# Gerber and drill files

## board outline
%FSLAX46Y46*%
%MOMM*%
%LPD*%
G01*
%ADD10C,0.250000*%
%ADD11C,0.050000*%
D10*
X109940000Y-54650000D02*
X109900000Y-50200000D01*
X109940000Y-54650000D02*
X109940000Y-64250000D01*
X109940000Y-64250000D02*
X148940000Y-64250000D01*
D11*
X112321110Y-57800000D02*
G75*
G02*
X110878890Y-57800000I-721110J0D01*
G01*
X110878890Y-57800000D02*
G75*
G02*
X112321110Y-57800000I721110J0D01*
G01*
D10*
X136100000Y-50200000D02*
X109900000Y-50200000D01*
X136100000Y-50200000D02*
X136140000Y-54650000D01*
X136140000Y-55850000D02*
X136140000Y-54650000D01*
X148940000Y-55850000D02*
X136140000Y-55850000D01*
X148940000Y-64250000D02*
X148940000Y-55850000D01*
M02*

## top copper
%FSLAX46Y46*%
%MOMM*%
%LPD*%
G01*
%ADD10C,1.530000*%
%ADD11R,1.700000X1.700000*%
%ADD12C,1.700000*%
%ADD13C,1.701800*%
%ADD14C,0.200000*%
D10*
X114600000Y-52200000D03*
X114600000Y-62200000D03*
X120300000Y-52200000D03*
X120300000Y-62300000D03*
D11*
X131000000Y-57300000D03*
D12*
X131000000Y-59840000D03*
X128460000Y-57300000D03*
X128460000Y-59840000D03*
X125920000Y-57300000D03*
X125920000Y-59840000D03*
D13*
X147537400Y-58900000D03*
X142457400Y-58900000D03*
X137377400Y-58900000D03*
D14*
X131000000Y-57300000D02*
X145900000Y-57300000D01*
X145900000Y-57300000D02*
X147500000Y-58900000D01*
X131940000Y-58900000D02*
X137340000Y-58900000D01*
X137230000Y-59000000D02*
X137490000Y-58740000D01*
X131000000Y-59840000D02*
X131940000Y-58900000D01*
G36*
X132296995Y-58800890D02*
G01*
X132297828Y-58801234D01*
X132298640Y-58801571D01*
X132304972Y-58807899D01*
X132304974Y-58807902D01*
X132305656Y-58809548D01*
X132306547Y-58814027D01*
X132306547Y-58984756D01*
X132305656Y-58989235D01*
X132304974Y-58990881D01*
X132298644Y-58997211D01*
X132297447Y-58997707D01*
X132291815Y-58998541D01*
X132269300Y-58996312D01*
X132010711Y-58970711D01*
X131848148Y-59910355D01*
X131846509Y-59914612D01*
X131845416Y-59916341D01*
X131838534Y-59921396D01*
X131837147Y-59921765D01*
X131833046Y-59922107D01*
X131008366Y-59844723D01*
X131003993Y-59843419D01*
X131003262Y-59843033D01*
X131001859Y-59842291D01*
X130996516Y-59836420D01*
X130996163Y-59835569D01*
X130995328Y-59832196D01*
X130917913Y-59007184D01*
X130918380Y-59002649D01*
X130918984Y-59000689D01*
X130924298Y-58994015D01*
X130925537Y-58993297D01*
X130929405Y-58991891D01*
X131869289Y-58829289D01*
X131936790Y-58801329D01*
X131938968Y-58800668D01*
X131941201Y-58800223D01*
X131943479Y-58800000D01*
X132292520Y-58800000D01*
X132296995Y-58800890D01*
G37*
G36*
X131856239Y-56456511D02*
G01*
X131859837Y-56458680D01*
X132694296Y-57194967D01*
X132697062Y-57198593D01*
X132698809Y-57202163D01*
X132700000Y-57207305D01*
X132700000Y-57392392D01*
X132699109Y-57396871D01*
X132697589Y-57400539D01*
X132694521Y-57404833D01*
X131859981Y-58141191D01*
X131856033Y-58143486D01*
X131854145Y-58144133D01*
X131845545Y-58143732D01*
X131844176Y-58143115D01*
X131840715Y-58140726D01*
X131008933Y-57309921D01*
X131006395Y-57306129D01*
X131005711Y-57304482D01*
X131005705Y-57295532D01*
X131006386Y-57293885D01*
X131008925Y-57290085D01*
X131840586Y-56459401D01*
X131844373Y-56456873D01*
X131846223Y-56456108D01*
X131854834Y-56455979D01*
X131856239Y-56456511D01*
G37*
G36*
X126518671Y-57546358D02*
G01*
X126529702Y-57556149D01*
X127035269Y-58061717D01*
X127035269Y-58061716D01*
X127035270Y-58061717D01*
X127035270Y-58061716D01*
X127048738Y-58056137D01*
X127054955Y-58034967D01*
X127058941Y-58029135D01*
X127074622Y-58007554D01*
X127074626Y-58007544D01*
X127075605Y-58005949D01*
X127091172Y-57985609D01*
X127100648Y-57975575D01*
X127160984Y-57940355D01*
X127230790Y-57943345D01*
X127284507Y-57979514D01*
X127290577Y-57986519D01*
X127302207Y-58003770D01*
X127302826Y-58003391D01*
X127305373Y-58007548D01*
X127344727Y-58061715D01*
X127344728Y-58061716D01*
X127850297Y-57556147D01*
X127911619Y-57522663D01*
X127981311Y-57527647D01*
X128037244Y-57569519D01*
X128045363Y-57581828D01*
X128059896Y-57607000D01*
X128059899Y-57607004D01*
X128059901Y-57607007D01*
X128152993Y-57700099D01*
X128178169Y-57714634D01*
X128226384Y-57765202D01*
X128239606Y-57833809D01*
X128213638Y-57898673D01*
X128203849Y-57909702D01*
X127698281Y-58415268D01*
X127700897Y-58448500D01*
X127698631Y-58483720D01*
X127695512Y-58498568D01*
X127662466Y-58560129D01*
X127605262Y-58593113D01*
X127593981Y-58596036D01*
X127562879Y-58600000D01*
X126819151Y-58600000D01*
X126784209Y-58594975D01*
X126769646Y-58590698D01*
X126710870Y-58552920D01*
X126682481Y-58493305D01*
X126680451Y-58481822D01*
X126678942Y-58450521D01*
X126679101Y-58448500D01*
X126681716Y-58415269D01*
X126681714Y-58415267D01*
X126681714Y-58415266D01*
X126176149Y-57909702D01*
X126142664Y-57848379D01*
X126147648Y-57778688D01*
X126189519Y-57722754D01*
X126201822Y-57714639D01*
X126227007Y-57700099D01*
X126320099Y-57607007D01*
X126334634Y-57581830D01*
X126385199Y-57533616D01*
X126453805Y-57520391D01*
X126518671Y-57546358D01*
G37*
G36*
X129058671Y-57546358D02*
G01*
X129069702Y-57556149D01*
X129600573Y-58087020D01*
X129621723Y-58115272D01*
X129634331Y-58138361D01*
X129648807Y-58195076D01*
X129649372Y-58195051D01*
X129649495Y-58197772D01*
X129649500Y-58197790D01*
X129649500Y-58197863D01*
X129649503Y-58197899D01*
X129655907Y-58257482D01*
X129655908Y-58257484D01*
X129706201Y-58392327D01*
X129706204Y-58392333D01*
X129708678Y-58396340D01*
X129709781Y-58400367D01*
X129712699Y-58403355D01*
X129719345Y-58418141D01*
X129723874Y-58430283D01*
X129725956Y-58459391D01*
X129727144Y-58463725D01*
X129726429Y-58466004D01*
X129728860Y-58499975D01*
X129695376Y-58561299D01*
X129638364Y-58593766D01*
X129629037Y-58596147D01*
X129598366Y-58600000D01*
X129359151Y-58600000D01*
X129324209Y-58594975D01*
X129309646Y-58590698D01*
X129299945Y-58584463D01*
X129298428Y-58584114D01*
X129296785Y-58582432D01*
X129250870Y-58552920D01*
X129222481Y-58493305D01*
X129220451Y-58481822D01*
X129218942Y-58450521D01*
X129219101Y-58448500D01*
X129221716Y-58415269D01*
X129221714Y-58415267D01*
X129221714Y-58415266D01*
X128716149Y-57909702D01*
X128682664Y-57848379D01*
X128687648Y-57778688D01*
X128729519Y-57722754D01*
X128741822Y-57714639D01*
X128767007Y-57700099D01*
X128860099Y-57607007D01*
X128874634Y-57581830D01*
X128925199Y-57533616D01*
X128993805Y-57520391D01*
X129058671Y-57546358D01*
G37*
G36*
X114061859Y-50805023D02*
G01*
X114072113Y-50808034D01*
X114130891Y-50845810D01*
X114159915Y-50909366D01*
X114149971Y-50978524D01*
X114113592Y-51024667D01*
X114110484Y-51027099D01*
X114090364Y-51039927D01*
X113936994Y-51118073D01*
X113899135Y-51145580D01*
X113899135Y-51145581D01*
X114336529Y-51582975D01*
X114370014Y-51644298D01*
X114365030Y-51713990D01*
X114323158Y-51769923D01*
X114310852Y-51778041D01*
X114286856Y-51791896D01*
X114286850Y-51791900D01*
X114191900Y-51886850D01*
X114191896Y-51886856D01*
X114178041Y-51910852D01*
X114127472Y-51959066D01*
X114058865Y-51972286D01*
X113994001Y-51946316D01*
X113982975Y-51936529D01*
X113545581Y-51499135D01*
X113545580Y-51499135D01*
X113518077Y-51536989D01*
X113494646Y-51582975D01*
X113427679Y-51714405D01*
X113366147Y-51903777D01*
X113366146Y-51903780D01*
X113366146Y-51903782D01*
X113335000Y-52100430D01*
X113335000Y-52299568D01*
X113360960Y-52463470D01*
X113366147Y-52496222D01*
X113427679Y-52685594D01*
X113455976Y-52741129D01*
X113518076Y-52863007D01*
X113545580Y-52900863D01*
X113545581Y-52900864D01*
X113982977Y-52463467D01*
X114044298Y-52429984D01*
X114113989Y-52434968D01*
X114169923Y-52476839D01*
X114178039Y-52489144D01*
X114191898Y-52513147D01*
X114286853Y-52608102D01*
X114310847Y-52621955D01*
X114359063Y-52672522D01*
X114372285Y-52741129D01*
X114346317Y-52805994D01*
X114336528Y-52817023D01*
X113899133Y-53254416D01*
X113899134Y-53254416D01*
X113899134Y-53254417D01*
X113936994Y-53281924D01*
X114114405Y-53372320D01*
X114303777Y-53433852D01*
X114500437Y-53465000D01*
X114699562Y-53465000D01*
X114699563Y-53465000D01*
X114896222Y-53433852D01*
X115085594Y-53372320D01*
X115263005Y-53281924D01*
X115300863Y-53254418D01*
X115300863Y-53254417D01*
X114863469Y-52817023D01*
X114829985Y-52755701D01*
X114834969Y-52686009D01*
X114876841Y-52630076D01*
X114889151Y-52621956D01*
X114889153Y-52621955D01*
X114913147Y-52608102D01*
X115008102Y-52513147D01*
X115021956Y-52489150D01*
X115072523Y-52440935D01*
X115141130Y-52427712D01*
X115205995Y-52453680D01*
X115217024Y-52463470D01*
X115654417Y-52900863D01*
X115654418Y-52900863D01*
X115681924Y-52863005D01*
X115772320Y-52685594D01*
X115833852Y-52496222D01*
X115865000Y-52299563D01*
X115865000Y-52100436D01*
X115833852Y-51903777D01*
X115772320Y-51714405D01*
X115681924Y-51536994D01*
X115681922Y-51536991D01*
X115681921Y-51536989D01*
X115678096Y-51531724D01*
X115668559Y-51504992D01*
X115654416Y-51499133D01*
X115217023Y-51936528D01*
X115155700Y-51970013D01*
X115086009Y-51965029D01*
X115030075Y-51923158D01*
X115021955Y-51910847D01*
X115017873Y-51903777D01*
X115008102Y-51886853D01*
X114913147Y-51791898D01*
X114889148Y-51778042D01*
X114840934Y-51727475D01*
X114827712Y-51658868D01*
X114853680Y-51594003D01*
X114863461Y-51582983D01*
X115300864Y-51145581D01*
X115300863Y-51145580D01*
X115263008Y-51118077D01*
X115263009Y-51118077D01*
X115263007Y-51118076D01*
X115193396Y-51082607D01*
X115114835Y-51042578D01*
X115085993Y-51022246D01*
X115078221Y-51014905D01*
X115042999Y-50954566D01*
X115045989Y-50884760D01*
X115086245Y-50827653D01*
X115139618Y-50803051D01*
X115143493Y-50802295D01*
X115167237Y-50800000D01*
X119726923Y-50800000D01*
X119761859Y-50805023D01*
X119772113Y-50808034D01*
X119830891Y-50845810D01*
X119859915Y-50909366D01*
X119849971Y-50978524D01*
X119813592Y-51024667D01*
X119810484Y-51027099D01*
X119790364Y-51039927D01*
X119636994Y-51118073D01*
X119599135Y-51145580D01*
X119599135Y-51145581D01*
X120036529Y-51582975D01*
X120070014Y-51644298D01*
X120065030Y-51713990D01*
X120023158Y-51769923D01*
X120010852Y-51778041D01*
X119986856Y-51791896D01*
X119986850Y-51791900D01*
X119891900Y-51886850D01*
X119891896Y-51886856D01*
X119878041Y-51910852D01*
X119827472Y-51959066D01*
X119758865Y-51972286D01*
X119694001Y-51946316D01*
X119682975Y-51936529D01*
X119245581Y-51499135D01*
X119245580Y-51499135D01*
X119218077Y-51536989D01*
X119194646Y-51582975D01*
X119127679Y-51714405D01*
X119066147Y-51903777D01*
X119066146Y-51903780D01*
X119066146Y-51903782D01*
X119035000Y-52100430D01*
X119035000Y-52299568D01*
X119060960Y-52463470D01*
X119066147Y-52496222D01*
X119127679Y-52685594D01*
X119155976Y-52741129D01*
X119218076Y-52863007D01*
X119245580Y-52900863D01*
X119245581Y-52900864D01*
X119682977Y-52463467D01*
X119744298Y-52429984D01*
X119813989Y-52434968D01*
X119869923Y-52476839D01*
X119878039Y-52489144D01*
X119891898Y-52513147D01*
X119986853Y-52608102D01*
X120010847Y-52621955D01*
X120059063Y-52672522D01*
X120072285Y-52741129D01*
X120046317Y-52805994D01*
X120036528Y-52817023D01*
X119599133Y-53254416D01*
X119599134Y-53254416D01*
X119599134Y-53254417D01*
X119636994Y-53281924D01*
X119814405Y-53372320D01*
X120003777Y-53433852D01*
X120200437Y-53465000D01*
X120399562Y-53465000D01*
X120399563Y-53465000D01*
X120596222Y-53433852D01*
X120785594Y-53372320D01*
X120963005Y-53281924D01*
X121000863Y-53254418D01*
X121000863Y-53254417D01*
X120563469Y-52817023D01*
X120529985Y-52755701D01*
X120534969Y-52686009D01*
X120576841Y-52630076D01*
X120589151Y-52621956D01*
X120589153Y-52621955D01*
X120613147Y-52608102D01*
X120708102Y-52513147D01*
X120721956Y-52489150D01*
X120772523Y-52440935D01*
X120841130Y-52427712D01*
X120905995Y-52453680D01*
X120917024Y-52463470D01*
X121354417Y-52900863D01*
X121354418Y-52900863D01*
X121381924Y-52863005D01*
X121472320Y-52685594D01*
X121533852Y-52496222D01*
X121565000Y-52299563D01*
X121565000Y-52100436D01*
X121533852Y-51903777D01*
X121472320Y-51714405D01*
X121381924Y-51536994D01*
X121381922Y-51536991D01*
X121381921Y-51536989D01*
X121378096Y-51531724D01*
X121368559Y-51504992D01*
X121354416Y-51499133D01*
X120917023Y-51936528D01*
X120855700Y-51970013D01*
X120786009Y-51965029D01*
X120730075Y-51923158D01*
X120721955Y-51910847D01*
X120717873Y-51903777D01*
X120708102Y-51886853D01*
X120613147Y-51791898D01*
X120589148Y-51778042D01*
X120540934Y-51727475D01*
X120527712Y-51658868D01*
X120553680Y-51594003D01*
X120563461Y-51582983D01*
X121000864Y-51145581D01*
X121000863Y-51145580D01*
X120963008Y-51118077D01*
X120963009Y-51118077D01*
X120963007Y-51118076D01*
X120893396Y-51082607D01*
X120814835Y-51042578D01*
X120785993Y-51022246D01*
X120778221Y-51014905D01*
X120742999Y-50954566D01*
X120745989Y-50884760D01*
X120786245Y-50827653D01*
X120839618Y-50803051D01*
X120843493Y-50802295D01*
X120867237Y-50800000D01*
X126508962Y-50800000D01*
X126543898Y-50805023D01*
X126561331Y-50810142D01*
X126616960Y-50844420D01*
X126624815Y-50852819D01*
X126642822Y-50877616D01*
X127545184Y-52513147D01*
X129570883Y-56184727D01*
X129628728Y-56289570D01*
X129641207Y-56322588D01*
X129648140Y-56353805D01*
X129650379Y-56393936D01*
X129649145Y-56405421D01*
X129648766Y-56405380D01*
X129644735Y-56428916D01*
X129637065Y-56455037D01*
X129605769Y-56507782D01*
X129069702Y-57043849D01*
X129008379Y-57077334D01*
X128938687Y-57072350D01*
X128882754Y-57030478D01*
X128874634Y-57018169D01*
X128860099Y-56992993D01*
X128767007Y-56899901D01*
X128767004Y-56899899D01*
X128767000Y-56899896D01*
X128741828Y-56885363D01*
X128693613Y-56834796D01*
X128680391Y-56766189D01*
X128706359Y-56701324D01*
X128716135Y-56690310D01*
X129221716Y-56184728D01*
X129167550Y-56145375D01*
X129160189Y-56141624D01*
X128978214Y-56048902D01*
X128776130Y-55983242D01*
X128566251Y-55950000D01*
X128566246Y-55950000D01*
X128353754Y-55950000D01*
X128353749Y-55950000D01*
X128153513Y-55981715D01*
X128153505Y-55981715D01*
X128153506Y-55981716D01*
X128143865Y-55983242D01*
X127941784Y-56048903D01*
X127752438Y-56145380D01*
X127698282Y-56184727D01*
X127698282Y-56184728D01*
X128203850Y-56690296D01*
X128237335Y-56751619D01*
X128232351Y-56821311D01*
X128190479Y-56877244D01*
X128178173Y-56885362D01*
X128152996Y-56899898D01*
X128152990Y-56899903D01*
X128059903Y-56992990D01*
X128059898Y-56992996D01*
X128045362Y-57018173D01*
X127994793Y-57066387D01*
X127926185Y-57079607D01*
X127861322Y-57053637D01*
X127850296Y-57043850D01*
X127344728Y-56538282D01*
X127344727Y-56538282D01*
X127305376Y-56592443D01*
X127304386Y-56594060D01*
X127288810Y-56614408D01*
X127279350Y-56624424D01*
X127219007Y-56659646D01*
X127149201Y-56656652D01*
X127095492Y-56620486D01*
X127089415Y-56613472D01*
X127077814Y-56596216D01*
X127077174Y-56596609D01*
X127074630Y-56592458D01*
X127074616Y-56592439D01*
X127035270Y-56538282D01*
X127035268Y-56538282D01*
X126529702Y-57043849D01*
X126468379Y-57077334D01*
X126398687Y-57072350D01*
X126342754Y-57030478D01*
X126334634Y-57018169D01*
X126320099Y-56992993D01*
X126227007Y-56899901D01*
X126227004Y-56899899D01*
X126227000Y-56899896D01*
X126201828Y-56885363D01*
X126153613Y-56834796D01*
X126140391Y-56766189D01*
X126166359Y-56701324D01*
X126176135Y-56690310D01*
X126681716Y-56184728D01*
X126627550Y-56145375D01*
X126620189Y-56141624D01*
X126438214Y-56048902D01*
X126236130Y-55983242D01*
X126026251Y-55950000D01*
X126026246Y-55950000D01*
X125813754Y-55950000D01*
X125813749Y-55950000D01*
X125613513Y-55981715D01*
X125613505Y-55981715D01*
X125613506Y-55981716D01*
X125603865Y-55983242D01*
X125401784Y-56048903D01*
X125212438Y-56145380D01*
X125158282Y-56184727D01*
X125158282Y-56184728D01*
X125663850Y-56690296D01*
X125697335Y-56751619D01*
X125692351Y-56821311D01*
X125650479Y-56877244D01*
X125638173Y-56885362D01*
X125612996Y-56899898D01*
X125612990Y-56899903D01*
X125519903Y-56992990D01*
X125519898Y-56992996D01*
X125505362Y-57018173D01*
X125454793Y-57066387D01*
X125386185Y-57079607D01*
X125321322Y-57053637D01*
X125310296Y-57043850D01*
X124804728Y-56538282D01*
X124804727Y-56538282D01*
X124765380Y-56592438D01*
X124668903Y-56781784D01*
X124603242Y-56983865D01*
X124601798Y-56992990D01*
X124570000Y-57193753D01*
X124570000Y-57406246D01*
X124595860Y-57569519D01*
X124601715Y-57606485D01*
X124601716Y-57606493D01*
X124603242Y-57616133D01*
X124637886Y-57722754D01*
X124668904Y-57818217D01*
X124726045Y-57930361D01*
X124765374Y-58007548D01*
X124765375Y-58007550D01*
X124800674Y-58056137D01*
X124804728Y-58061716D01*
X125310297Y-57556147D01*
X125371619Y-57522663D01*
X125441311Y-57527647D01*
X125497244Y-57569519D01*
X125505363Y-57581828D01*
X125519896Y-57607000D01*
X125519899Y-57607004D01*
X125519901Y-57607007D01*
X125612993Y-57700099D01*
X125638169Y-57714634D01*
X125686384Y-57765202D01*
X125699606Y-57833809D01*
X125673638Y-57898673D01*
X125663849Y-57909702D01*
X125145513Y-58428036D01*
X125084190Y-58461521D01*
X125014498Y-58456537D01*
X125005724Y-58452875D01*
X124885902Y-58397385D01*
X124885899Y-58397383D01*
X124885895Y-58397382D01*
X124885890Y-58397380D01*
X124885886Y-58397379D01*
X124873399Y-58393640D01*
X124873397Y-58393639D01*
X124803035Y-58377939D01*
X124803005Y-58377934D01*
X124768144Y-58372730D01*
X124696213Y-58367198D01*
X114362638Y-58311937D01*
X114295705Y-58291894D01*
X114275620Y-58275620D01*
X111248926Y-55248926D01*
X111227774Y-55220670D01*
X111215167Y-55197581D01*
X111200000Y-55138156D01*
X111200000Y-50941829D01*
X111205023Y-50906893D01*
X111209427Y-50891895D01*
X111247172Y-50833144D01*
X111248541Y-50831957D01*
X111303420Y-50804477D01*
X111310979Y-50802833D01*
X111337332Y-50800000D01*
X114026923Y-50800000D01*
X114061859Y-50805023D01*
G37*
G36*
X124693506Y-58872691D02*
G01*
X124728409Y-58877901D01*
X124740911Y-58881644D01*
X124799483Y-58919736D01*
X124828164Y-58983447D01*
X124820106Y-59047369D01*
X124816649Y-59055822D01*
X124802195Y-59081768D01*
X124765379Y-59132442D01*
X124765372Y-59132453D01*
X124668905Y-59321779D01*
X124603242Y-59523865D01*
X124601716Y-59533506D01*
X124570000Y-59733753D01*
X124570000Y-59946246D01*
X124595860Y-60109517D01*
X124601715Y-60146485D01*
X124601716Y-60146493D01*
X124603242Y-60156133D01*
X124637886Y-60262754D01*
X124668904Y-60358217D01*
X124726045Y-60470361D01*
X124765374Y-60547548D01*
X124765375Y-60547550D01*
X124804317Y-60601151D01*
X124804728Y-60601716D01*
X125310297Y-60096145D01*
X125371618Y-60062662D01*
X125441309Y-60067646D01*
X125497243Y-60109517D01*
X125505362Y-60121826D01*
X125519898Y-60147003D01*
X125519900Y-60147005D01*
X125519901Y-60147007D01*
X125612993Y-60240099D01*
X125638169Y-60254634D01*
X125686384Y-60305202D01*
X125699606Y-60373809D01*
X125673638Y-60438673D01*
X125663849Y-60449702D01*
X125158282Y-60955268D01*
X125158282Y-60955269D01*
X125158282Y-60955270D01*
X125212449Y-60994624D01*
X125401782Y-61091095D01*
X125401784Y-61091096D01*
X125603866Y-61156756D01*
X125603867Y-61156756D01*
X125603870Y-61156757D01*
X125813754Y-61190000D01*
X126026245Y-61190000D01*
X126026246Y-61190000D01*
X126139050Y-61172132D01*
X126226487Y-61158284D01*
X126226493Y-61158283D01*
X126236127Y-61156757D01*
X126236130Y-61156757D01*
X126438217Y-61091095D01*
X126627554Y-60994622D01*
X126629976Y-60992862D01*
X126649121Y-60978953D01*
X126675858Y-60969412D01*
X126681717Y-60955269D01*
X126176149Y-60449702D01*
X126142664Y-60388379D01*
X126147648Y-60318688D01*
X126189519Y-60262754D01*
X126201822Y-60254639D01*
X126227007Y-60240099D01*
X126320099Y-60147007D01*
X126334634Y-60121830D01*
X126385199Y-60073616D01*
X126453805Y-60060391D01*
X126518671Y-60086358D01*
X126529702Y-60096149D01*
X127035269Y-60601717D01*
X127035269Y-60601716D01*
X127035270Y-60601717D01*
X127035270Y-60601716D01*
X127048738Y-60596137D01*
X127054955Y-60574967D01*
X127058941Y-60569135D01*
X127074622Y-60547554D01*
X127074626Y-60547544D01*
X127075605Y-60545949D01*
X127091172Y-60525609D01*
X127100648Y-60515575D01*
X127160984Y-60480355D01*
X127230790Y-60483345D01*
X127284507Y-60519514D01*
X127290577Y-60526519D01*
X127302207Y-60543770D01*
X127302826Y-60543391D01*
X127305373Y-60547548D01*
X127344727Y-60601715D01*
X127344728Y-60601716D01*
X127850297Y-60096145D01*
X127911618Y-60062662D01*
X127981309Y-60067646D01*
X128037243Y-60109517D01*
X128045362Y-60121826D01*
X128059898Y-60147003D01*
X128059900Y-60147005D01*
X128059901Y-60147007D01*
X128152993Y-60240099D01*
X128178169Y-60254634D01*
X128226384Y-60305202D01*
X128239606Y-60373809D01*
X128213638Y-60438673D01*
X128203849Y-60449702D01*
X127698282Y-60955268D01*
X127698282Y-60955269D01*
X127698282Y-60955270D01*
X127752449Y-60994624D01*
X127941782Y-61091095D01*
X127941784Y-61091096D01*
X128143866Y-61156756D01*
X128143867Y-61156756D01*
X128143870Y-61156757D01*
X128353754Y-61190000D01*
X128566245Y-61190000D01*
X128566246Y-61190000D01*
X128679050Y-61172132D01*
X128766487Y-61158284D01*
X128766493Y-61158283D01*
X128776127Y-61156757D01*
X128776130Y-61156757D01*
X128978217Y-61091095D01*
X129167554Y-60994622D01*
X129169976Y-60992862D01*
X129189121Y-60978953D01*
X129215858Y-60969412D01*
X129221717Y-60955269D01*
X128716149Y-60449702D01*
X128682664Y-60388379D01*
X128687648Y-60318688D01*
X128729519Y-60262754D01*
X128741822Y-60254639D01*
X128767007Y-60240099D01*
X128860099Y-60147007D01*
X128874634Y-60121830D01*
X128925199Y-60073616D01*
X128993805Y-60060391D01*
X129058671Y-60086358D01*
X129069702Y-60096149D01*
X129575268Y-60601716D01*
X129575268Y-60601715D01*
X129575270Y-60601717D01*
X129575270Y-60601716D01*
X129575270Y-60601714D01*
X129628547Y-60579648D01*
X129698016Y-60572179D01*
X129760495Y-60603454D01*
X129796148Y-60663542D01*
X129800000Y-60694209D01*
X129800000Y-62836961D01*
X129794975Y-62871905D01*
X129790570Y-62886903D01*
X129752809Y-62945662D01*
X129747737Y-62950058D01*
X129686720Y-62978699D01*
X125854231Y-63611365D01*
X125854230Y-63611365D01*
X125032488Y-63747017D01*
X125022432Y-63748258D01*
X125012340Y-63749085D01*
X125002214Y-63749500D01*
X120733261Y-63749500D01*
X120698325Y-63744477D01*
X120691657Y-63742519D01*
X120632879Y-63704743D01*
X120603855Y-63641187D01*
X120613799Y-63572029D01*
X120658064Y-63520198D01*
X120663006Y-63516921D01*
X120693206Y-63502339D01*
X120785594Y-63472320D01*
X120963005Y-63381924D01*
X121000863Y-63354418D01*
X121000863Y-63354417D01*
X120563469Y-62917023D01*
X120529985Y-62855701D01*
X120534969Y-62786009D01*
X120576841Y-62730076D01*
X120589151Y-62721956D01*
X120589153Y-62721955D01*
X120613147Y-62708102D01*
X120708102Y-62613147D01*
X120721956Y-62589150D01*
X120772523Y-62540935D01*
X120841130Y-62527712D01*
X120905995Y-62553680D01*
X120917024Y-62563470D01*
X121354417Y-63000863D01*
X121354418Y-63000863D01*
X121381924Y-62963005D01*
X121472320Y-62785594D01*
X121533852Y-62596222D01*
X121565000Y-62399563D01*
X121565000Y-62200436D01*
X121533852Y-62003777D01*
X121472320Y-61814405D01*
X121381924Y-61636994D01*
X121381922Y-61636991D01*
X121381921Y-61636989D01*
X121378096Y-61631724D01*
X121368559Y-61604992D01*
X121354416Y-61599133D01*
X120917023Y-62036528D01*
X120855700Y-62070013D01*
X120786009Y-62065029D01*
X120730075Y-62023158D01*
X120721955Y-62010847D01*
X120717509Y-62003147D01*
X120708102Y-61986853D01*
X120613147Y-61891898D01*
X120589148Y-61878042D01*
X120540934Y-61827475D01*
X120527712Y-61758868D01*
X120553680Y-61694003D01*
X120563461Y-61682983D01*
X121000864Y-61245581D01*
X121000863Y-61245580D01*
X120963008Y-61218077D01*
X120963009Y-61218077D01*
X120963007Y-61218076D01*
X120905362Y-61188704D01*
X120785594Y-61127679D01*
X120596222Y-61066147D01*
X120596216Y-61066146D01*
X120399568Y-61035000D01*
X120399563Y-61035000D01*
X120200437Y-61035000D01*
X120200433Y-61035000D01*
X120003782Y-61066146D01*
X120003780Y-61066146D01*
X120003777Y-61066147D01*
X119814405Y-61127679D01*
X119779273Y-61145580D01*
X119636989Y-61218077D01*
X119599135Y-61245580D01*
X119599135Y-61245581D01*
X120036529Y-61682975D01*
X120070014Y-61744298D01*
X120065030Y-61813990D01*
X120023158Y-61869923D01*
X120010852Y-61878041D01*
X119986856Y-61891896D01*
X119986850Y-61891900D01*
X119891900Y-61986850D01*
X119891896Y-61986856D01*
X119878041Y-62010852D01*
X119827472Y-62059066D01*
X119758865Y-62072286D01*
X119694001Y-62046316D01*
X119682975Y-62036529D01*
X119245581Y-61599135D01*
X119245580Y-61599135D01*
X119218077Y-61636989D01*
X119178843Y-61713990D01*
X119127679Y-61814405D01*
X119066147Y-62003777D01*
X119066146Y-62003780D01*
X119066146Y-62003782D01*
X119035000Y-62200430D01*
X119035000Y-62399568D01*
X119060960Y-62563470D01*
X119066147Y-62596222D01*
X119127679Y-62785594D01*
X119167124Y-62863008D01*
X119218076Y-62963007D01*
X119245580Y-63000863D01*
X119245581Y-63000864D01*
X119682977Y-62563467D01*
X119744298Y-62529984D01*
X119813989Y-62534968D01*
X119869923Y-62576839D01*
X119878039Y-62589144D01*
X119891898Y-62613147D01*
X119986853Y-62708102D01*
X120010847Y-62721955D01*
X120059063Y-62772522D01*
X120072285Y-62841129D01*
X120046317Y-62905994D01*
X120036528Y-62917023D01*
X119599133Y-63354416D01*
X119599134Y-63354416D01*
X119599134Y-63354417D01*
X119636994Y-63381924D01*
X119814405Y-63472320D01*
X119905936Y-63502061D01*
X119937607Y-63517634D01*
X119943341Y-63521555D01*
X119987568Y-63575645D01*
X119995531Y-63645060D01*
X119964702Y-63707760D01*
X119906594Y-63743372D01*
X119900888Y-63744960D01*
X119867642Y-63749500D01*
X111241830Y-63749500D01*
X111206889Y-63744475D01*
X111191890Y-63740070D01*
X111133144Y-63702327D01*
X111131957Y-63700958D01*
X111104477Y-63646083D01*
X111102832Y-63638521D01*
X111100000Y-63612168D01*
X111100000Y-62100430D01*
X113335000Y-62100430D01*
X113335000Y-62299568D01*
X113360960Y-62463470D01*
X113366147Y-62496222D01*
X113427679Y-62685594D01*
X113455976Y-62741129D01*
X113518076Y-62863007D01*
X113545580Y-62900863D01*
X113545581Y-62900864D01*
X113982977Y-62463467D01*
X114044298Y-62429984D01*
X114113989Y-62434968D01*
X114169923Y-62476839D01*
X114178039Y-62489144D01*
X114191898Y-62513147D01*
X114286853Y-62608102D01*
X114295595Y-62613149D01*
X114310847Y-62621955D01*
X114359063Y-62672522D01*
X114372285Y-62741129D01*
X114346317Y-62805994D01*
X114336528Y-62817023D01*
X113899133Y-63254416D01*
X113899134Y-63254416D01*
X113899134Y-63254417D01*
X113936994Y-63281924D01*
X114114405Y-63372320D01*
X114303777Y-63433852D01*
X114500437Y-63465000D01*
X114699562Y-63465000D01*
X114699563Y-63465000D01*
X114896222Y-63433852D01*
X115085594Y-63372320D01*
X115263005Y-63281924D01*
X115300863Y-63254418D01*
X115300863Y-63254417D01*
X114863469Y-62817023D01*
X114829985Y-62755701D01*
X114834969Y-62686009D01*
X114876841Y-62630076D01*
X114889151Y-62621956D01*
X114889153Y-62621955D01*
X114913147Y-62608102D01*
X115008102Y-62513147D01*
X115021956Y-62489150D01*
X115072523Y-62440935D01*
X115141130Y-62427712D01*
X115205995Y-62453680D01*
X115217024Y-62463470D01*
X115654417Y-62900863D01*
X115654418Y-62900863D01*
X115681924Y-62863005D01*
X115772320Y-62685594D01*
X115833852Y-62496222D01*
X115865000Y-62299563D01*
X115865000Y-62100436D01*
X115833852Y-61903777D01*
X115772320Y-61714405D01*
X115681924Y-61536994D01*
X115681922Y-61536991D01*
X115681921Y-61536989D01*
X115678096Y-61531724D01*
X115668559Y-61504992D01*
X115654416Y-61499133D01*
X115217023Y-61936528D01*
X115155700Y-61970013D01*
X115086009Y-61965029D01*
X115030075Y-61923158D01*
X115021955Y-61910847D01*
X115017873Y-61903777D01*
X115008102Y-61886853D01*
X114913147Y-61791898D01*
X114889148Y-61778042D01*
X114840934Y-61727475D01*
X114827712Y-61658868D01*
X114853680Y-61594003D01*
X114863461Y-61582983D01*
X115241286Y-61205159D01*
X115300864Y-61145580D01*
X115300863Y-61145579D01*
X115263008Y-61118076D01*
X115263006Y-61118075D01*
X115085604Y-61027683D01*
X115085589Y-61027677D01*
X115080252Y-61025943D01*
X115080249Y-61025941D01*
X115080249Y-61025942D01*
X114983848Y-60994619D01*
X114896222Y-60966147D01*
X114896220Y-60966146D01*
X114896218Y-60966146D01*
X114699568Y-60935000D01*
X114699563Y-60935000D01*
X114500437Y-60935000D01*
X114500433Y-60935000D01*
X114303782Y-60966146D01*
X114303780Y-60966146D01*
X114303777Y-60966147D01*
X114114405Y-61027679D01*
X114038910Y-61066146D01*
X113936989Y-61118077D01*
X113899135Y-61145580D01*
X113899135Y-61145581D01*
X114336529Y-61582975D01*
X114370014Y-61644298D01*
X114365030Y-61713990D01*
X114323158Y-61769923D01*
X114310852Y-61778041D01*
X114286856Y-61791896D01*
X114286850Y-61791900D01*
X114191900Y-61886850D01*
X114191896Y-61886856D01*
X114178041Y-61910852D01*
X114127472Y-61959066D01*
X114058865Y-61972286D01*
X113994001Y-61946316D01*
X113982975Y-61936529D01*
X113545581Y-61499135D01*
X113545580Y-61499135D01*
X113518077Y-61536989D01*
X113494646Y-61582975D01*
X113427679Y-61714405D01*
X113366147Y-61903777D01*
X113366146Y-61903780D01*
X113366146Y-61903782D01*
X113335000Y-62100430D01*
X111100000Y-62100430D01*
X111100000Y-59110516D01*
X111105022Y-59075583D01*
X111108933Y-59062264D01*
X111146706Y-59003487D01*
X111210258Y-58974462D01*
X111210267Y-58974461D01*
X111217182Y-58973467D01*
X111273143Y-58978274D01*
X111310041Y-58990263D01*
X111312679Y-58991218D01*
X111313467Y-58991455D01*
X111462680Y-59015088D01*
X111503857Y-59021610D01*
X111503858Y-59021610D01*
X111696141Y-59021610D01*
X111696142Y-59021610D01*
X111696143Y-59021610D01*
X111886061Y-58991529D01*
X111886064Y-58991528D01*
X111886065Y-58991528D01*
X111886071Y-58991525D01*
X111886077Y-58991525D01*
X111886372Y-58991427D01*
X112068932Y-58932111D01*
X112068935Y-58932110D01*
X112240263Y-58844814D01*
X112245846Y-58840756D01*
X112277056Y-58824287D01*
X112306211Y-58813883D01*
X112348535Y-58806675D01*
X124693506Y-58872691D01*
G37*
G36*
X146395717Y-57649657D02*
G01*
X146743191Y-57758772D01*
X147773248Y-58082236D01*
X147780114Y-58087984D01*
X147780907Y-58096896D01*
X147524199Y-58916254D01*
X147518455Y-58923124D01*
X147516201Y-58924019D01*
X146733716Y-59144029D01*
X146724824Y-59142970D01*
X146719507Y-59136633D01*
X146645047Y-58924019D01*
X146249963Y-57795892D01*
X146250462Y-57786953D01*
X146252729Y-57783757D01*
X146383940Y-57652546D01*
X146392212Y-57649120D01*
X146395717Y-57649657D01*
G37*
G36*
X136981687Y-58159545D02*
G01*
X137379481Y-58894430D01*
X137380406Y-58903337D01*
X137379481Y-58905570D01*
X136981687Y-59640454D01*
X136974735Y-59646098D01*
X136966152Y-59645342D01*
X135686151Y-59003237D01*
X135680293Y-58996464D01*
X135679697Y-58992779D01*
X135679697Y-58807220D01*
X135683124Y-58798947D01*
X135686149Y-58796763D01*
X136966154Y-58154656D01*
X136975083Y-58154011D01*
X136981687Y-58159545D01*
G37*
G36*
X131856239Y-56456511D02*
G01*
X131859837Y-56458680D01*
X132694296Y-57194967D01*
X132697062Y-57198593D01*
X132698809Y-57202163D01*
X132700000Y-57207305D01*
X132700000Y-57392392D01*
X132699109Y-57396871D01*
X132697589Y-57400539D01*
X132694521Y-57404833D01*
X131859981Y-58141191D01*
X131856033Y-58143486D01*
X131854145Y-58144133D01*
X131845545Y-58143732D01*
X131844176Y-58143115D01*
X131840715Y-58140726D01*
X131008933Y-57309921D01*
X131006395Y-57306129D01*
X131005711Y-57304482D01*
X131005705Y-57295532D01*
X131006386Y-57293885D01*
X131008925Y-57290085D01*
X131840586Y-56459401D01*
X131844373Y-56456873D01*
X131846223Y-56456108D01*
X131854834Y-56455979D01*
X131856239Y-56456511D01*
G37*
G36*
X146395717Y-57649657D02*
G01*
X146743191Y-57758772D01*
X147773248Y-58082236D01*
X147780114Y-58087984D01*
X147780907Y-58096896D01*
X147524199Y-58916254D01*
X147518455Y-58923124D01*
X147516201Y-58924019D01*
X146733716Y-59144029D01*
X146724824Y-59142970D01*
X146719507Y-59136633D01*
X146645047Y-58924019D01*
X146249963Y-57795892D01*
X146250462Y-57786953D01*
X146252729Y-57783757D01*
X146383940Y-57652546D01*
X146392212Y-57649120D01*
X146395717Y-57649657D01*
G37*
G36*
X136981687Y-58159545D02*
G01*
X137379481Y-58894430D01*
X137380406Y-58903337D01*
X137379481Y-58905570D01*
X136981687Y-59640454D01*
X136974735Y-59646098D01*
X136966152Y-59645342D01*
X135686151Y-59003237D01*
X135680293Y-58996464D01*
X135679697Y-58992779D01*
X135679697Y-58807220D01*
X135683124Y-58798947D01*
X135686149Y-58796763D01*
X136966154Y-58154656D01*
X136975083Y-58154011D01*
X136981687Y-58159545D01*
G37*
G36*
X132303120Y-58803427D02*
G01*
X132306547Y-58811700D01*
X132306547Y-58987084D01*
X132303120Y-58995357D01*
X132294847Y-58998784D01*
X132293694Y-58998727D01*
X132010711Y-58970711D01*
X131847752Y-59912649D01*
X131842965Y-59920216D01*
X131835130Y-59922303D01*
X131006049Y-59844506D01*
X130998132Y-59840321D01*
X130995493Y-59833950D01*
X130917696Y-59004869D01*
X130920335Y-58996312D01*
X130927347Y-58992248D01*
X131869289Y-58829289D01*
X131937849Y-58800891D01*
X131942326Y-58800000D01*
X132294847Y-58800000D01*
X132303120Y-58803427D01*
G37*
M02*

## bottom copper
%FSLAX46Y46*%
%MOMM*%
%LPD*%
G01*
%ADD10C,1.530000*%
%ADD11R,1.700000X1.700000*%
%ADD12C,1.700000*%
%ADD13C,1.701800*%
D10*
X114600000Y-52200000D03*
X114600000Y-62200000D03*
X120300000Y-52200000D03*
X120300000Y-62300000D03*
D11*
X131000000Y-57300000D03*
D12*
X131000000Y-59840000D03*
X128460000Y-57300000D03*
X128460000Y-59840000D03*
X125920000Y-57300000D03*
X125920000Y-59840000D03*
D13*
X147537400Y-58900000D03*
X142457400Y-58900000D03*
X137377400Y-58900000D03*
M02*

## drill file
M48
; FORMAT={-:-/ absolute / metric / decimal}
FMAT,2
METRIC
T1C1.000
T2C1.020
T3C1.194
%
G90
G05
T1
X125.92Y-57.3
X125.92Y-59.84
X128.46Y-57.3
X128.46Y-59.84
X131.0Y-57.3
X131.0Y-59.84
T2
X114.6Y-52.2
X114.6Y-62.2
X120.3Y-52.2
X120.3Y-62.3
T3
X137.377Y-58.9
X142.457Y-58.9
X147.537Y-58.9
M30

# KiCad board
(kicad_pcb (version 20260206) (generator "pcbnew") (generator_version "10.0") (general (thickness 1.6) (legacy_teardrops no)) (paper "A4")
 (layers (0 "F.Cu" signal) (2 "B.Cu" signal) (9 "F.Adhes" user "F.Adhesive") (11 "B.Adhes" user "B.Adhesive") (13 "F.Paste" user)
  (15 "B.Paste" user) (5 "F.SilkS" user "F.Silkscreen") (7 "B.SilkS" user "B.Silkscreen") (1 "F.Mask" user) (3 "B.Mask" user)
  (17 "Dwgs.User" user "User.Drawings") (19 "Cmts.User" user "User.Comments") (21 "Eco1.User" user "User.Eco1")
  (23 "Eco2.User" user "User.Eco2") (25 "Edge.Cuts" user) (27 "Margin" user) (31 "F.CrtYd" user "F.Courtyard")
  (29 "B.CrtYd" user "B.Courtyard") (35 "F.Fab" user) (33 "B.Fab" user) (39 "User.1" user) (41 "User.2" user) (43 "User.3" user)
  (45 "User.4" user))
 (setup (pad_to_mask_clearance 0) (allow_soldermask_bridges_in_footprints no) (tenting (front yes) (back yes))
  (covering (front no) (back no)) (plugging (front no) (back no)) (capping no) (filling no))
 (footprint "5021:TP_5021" (layer "F.Cu") (at 114.6 52.2 -90)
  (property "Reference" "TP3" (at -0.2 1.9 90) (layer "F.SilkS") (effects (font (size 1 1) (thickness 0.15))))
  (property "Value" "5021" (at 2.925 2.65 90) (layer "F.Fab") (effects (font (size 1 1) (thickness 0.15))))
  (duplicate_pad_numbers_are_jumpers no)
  (pad "TP" thru_hole circle (at 0 0 270) (size 1.53 1.53) (drill 1.02) (layers "*.Cu" "*.Mask") (remove_unused_layers no)
   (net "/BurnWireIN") (solder_mask_margin 0.102)
   (teardrops (best_length_ratio 0.5) (max_length 1) (best_width_ratio 1) (max_width 2) (curved_edges no) (filter_ratio 0.9) (enabled yes)
    (allow_two_segments yes) (prefer_zone_connections yes))))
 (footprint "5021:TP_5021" (layer "F.Cu") (at 114.6 62.2 -90)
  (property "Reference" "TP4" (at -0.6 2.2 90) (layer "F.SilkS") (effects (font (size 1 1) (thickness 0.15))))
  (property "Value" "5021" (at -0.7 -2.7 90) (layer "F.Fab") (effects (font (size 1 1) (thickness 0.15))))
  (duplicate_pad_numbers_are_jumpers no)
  (pad "TP" thru_hole circle (at 0 0 270) (size 1.53 1.53) (drill 1.02) (layers "*.Cu" "*.Mask") (remove_unused_layers no) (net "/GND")
   (solder_mask_margin 0.102)
   (teardrops (best_length_ratio 0.5) (max_length 1) (best_width_ratio 1) (max_width 2) (curved_edges no) (filter_ratio 0.9) (enabled yes)
    (allow_two_segments yes) (prefer_zone_connections yes))))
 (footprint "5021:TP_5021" (layer "F.Cu") (at 120.3 52.2 -90)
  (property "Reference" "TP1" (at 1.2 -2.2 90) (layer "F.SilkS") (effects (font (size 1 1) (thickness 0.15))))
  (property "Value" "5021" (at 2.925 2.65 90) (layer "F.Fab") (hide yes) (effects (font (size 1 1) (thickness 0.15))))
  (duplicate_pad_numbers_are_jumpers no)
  (pad "TP" thru_hole circle (at 0 0 270) (size 1.53 1.53) (drill 1.02) (layers "*.Cu" "*.Mask") (remove_unused_layers no)
   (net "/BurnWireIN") (solder_mask_margin 0.102)
   (teardrops (best_length_ratio 0.5) (max_length 1) (best_width_ratio 1) (max_width 2) (curved_edges no) (filter_ratio 0.9) (enabled yes)
    (allow_two_segments yes) (prefer_zone_connections yes))))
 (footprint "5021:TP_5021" (layer "F.Cu") (at 120.3 62.3 -90)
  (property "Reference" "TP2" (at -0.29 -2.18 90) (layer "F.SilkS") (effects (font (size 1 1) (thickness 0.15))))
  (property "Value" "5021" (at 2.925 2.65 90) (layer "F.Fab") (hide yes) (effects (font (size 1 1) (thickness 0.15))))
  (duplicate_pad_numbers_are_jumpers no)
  (pad "TP" thru_hole circle (at 0 0 270) (size 1.53 1.53) (drill 1.02) (layers "*.Cu" "*.Mask") (remove_unused_layers no) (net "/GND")
   (solder_mask_margin 0.102)
   (teardrops (best_length_ratio 0.5) (max_length 1) (best_width_ratio 1) (max_width 2) (curved_edges no) (filter_ratio 0.9) (enabled yes)
    (allow_two_segments yes) (prefer_zone_connections yes))))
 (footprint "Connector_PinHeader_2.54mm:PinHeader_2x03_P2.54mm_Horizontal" (layer "F.Cu") (at 131 57.3 -90)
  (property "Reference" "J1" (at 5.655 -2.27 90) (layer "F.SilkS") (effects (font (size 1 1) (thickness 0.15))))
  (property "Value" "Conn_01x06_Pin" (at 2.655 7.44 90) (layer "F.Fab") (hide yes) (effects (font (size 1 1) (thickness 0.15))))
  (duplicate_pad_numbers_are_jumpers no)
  (pad "1" thru_hole rect (at 0 0 270) (size 1.7 1.7) (drill 1) (layers "*.Cu" "*.Mask") (remove_unused_layers no)
   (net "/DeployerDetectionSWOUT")
   (teardrops (best_length_ratio 0.5) (max_length 1) (best_width_ratio 1) (max_width 2) (curved_edges no) (filter_ratio 0.9) (enabled yes)
    (allow_two_segments yes) (prefer_zone_connections yes)))
  (pad "2" thru_hole circle (at 2.54 0 270) (size 1.7 1.7) (drill 1) (layers "*.Cu" "*.Mask") (remove_unused_layers no)
   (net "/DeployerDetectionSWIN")
   (teardrops (best_length_ratio 0.5) (max_length 1) (best_width_ratio 1) (max_width 2) (curved_edges no) (filter_ratio 0.9) (enabled yes)
    (allow_two_segments yes) (prefer_zone_connections yes)))
  (pad "3" thru_hole circle (at 0 2.54 270) (size 1.7 1.7) (drill 1) (layers "*.Cu" "*.Mask") (remove_unused_layers no) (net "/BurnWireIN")
   (teardrops (best_length_ratio 0.5) (max_length 1) (best_width_ratio 1) (max_width 2) (curved_edges no) (filter_ratio 0.9) (enabled yes)
    (allow_two_segments yes) (prefer_zone_connections yes)))
  (pad "4" thru_hole circle (at 2.54 2.54 270) (size 1.7 1.7) (drill 1) (layers "*.Cu" "*.Mask") (remove_unused_layers no) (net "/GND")
   (teardrops (best_length_ratio 0.5) (max_length 1) (best_width_ratio 1) (max_width 2) (curved_edges no) (filter_ratio 0.9) (enabled yes)
    (allow_two_segments yes) (prefer_zone_connections yes)))
  (pad "5" thru_hole circle (at 0 5.08 270) (size 1.7 1.7) (drill 1) (layers "*.Cu" "*.Mask") (remove_unused_layers no) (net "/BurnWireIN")
   (teardrops (best_length_ratio 0.5) (max_length 1) (best_width_ratio 1) (max_width 2) (curved_edges no) (filter_ratio 0.9) (enabled yes)
    (allow_two_segments yes) (prefer_zone_connections yes)))
  (pad "6" thru_hole circle (at 2.54 5.08 270) (size 1.7 1.7) (drill 1) (layers "*.Cu" "*.Mask") (remove_unused_layers no) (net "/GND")
   (teardrops (best_length_ratio 0.5) (max_length 1) (best_width_ratio 1) (max_width 2) (curved_edges no) (filter_ratio 0.9) (enabled yes)
    (allow_two_segments yes) (prefer_zone_connections yes))))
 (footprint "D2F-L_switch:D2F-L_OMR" (layer "B.Cu") (at 147.5374 58.9 180)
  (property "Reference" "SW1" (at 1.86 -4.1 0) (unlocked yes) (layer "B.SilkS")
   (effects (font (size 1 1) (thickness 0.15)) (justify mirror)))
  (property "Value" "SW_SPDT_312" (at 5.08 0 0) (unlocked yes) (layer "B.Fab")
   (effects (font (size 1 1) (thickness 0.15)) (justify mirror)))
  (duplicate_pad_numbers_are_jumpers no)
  (pad "1" thru_hole circle (at 0 0 180) (size 1.7018 1.7018) (drill 1.1938) (layers "*.Cu" "*.Mask") (remove_unused_layers no)
   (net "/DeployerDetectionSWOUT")
   (teardrops (best_length_ratio 0.5) (max_length 1) (best_width_ratio 1) (max_width 2) (curved_edges no) (filter_ratio 0.9) (enabled yes)
    (allow_two_segments yes) (prefer_zone_connections yes)))
  (pad "2" thru_hole circle (at 5.08 0 180) (size 1.7018 1.7018) (drill 1.1938) (layers "*.Cu" "*.Mask") (remove_unused_layers no)
   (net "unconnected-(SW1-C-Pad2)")
   (teardrops (best_length_ratio 0.5) (max_length 1) (best_width_ratio 1) (max_width 2) (curved_edges no) (filter_ratio 0.9) (enabled yes)
    (allow_two_segments yes) (prefer_zone_connections yes)))
  (pad "3" thru_hole circle (at 10.16 0 180) (size 1.7018 1.7018) (drill 1.1938) (layers "*.Cu" "*.Mask") (remove_unused_layers no)
   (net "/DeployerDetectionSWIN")
   (teardrops (best_length_ratio 0.5) (max_length 1) (best_width_ratio 1) (max_width 2) (curved_edges no) (filter_ratio 0.9) (enabled yes)
    (allow_two_segments yes) (prefer_zone_connections yes))))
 (gr_line (start 109.94 54.65) (end 109.9 50.2) (stroke (width 0.25) (type solid)) (layer "Edge.Cuts"))
 (gr_line (start 109.94 54.65) (end 109.94 64.25) (stroke (width 0.25) (type default)) (layer "Edge.Cuts"))
 (gr_line (start 109.94 64.25) (end 148.94 64.25) (stroke (width 0.25) (type solid)) (layer "Edge.Cuts"))
 (gr_circle (center 111.6 57.8) (end 112.2 58.2) (stroke (width 0.05) (type default)) (fill no) (layer "Edge.Cuts"))
 (gr_line (start 136.1 50.2) (end 109.9 50.2) (stroke (width 0.25) (type default)) (layer "Edge.Cuts"))
 (gr_line (start 136.1 50.2) (end 136.14 54.65) (stroke (width 0.25) (type solid)) (layer "Edge.Cuts"))
 (gr_line (start 136.14 55.85) (end 136.14 54.65) (stroke (width 0.25) (type default)) (layer "Edge.Cuts"))
 (gr_line (start 148.94 55.85) (end 136.14 55.85) (stroke (width 0.25) (type default)) (layer "Edge.Cuts"))
 (gr_line (start 148.94 64.25) (end 148.94 55.85) (stroke (width 0.25) (type default)) (layer "Edge.Cuts"))
 (segment (start 131 57.3) (end 145.9 57.3) (width 0.2) (layer "F.Cu") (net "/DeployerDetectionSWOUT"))
 (segment (start 145.9 57.3) (end 147.5 58.9) (width 0.2) (layer "F.Cu") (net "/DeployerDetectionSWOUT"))
 (segment (start 131.94 58.9) (end 137.34 58.9) (width 0.2) (layer "F.Cu") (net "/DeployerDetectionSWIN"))
 (segment (start 137.23 59) (end 137.49 58.74) (width 0.2) (layer "F.Cu") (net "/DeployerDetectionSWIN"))
 (segment (start 131 59.84) (end 131.94 58.9) (width 0.2) (layer "F.Cu") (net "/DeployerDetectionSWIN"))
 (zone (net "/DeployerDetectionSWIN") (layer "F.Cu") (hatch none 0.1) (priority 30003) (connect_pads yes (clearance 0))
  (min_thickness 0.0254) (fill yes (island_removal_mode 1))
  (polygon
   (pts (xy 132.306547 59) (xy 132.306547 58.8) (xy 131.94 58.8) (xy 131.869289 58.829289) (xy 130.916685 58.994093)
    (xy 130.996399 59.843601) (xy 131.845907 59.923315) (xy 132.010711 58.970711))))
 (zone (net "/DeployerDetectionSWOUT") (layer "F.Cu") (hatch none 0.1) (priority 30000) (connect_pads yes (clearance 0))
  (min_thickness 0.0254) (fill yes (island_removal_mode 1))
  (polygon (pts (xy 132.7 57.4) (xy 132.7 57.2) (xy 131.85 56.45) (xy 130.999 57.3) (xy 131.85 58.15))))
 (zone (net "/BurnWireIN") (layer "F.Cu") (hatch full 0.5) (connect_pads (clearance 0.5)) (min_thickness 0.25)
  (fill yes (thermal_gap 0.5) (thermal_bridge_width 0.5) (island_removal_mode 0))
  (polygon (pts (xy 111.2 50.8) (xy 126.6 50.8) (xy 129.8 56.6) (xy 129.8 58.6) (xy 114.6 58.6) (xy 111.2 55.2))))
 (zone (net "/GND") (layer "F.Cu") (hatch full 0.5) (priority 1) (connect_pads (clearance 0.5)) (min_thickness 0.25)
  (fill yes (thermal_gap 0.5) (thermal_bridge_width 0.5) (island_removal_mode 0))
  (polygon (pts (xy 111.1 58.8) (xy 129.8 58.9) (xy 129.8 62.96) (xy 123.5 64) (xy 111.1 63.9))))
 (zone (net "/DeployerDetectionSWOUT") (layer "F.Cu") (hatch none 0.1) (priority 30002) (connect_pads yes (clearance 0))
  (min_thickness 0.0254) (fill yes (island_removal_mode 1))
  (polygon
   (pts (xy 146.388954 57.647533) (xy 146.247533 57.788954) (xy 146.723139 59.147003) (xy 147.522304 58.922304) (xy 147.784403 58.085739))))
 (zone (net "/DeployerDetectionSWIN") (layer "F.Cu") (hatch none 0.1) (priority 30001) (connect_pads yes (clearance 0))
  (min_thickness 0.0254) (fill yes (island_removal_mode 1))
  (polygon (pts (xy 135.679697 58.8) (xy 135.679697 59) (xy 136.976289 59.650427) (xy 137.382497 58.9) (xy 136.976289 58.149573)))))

